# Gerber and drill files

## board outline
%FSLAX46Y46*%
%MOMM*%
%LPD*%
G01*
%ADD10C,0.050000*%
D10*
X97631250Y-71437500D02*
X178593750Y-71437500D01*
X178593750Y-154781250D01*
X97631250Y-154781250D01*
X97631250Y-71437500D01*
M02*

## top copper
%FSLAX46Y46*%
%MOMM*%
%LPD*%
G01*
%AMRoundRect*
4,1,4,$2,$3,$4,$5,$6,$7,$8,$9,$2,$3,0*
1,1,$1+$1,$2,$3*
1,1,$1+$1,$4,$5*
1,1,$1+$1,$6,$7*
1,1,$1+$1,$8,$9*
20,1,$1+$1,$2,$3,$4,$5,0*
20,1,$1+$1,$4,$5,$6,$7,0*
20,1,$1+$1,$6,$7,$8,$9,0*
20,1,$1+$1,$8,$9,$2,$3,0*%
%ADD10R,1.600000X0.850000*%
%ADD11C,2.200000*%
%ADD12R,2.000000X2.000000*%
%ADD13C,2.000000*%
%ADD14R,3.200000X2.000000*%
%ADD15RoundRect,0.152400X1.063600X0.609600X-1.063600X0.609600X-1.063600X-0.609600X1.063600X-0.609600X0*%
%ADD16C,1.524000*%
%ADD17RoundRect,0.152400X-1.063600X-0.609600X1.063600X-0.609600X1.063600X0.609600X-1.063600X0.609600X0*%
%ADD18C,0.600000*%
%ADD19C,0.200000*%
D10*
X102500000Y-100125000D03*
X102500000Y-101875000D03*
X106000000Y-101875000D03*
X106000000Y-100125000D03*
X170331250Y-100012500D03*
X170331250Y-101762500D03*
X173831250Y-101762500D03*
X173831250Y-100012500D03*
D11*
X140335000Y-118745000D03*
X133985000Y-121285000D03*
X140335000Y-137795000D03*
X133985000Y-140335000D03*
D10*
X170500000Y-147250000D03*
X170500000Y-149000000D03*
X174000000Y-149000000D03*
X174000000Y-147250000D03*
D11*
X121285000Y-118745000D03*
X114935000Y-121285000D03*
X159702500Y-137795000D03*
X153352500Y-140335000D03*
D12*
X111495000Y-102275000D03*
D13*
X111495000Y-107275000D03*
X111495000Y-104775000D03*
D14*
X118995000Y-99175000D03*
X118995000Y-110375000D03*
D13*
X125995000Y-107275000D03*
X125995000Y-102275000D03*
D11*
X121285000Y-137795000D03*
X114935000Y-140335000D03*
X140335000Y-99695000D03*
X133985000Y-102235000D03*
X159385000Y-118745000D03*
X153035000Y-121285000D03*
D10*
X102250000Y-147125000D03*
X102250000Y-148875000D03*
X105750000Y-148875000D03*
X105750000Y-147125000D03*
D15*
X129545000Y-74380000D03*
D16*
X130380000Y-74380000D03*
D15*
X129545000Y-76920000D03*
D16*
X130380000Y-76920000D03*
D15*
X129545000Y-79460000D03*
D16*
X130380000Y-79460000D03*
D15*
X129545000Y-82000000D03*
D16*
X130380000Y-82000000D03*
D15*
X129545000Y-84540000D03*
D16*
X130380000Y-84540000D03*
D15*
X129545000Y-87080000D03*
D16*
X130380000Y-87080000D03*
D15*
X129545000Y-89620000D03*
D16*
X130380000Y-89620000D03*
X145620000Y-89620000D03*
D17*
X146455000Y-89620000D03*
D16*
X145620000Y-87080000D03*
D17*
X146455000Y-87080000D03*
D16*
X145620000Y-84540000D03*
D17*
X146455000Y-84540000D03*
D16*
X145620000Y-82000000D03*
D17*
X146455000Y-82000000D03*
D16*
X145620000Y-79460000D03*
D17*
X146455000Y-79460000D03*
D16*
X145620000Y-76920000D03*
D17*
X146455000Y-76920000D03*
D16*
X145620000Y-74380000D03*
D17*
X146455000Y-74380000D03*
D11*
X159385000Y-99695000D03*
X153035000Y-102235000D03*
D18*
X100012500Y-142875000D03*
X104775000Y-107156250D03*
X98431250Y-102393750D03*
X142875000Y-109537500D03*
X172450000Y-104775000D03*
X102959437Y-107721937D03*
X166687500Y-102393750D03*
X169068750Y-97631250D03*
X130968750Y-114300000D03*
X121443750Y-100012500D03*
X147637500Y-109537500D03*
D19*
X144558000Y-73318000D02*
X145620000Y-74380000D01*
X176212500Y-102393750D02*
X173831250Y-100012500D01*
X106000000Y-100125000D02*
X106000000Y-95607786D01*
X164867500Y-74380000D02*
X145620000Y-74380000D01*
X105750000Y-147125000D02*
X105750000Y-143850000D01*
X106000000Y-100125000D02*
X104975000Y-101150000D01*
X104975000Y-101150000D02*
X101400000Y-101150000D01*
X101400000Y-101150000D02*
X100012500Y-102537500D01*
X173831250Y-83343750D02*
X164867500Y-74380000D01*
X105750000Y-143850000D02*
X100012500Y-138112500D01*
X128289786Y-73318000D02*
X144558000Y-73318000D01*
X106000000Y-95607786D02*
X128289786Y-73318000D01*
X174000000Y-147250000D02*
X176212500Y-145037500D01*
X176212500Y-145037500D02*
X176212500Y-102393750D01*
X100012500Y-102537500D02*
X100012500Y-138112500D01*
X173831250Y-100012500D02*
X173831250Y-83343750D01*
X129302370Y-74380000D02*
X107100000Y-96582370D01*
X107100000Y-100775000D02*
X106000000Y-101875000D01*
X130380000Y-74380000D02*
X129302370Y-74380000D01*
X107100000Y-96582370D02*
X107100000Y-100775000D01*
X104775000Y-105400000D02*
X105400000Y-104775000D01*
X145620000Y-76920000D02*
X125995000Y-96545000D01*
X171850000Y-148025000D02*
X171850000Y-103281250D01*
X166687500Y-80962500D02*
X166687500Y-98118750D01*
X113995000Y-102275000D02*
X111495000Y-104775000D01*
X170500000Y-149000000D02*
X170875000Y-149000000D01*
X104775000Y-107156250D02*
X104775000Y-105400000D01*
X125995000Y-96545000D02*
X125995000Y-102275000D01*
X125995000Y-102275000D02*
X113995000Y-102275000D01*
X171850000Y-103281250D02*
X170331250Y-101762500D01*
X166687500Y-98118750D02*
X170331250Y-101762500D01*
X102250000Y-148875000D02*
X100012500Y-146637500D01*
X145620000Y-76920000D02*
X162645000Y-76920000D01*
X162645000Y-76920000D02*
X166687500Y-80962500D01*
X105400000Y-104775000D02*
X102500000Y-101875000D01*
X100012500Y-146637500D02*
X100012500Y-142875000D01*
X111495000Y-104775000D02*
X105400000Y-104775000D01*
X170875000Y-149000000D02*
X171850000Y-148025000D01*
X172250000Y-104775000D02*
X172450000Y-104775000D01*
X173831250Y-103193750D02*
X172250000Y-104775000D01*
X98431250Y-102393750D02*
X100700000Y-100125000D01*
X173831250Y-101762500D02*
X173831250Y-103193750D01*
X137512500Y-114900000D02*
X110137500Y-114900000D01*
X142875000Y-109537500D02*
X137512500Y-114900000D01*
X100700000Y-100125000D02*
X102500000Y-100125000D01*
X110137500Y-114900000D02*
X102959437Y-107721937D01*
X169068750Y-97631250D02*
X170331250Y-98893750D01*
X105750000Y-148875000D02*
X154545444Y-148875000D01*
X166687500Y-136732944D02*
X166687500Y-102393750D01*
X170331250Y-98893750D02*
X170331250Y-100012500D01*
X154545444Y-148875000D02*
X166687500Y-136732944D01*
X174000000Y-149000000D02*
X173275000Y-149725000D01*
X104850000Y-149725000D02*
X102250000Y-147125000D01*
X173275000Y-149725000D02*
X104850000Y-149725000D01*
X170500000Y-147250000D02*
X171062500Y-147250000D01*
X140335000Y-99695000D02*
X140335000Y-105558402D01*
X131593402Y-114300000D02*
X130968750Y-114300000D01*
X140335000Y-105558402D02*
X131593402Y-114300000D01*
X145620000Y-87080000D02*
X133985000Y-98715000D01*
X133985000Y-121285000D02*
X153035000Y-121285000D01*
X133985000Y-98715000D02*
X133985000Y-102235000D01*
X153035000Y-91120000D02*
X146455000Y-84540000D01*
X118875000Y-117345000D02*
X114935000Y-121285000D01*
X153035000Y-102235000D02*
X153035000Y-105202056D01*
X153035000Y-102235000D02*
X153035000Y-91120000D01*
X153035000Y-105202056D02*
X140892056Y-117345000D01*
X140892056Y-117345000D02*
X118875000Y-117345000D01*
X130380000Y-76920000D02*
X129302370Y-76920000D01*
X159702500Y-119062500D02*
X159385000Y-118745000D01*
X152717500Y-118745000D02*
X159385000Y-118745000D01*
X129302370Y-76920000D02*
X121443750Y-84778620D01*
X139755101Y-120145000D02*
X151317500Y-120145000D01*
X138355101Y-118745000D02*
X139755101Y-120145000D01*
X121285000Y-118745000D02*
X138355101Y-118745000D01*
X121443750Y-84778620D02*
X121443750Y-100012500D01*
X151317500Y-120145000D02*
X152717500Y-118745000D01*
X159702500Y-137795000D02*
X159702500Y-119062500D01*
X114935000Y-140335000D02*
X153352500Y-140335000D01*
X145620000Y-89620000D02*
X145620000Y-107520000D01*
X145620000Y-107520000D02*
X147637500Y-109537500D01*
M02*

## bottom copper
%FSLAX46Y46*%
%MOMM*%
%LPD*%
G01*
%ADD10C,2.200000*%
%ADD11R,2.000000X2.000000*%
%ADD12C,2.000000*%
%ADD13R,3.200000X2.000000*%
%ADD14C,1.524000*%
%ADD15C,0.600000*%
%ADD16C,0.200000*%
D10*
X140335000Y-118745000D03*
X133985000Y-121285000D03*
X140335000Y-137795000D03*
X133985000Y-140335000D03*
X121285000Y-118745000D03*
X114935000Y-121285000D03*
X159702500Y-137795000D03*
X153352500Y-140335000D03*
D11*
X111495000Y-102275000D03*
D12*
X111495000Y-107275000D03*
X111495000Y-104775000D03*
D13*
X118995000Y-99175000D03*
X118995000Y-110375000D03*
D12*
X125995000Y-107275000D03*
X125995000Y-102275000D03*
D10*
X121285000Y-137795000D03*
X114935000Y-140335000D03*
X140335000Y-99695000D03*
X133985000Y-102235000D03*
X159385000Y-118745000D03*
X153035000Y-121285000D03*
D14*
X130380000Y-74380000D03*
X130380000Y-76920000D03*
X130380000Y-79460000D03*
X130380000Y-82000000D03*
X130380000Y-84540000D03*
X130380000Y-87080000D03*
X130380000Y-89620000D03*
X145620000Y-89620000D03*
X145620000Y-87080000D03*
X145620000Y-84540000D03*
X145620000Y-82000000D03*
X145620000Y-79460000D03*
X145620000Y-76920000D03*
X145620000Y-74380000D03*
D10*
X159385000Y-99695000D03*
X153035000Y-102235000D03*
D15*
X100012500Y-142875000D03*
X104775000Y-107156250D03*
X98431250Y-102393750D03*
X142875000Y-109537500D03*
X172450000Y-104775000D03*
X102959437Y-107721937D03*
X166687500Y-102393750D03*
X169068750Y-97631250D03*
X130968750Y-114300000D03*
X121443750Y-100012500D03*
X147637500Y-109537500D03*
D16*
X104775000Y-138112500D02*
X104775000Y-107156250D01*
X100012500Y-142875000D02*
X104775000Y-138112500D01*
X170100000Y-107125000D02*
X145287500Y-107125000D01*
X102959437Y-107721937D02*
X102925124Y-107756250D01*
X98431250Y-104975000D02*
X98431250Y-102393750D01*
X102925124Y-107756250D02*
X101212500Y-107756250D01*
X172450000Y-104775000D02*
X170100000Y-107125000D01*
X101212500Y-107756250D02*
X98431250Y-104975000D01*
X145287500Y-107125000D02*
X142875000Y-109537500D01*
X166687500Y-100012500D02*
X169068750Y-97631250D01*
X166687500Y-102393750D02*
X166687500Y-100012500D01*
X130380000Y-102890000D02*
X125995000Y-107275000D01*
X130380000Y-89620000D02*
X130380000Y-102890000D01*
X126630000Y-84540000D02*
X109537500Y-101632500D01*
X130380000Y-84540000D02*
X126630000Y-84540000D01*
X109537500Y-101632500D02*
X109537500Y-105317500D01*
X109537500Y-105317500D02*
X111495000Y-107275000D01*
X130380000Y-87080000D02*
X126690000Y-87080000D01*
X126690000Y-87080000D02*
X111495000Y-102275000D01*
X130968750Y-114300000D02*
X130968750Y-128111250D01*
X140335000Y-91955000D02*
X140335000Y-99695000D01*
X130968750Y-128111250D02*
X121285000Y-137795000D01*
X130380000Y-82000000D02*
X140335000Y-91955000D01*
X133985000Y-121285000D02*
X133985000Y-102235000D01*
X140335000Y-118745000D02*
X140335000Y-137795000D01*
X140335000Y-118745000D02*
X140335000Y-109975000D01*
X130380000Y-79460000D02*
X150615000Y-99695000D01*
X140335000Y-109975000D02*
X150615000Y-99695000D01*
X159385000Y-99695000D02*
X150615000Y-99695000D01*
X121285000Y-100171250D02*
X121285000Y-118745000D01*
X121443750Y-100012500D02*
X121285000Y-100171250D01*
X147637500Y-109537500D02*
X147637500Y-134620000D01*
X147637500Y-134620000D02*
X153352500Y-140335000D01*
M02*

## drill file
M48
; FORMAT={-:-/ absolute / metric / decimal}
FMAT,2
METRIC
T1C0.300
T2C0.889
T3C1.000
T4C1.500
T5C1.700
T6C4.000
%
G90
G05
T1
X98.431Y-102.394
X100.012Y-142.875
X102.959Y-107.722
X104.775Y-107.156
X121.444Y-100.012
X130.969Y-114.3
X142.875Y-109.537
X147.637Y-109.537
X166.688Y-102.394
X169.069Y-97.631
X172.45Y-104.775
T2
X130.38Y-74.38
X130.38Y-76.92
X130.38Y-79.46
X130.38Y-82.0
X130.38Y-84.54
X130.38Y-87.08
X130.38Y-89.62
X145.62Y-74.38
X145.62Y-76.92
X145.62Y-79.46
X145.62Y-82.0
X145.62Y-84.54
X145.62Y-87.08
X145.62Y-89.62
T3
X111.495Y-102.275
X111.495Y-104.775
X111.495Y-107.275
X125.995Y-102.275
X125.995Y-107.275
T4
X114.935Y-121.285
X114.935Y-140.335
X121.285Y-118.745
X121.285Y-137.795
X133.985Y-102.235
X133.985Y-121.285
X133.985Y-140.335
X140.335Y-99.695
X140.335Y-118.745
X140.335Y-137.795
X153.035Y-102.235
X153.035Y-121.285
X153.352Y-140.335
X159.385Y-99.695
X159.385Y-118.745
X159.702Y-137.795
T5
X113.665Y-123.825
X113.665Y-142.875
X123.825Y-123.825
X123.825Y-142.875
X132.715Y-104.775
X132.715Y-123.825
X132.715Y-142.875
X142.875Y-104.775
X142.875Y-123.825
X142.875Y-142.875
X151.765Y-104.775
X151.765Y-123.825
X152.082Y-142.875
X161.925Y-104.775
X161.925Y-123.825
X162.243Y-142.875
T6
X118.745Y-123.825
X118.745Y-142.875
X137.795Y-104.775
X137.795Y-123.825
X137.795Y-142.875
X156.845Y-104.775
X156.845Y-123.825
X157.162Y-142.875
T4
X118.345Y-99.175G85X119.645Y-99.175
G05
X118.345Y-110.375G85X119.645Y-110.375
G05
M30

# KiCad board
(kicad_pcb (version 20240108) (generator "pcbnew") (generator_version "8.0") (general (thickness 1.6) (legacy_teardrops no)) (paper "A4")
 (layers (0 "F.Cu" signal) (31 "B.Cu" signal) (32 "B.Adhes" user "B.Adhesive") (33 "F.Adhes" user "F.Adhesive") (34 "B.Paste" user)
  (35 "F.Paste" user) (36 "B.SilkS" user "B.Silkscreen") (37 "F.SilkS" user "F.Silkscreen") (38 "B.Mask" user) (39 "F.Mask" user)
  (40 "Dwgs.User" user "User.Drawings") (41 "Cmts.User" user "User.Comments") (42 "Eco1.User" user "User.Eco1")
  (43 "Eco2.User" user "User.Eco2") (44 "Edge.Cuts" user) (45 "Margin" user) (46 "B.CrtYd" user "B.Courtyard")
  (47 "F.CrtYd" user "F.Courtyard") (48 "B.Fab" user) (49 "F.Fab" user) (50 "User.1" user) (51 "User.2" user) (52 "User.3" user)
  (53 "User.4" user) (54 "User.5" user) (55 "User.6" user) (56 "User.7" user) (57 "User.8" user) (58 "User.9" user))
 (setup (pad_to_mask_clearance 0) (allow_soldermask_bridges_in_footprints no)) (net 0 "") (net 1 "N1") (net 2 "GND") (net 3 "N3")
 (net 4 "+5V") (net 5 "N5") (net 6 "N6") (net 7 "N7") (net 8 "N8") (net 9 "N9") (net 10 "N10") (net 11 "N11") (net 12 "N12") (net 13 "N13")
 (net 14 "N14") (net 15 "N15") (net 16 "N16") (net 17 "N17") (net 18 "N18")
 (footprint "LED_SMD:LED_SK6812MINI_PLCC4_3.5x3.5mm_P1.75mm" (layer "F.Cu") (at 104.25 101)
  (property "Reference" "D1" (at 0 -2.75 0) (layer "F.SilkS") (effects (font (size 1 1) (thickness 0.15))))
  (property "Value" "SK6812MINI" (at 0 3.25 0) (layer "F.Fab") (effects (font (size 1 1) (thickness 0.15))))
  (pad "1" smd rect (at -1.75 -0.875) (size 1.6 0.85) (layers "F.Cu" "F.Paste" "F.Mask") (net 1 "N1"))
  (pad "2" smd rect (at -1.75 0.875) (size 1.6 0.85) (layers "F.Cu" "F.Paste" "F.Mask") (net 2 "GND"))
  (pad "3" smd rect (at 1.75 0.875) (size 1.6 0.85) (layers "F.Cu" "F.Paste" "F.Mask") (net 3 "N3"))
  (pad "4" smd rect (at 1.75 -0.875) (size 1.6 0.85) (layers "F.Cu" "F.Paste" "F.Mask") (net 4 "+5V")))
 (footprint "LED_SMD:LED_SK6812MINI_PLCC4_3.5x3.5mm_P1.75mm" (layer "F.Cu") (at 172.08125 100.8875)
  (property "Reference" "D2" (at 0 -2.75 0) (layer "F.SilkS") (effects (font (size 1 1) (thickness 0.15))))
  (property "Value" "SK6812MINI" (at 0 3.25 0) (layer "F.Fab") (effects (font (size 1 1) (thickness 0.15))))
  (pad "1" smd rect (at -1.75 -0.875) (size 1.6 0.85) (layers "F.Cu" "F.Paste" "F.Mask") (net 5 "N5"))
  (pad "2" smd rect (at -1.75 0.875) (size 1.6 0.85) (layers "F.Cu" "F.Paste" "F.Mask") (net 2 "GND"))
  (pad "3" smd rect (at 1.75 0.875) (size 1.6 0.85) (layers "F.Cu" "F.Paste" "F.Mask") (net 1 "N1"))
  (pad "4" smd rect (at 1.75 -0.875) (size 1.6 0.85) (layers "F.Cu" "F.Paste" "F.Mask") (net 4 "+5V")))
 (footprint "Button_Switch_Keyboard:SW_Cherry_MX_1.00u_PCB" (layer "F.Cu") (at 140.335 118.745)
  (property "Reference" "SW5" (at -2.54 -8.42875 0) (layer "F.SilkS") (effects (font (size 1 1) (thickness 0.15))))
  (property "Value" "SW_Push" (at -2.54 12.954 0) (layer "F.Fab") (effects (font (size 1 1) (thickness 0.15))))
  (pad "" np_thru_hole circle (at -7.62 5.08) (size 1.7 1.7) (drill 1.7) (layers "*.Cu" "*.Mask"))
  (pad "" np_thru_hole circle (at -2.54 5.08) (size 4 4) (drill 4) (layers "*.Cu" "*.Mask"))
  (pad "" np_thru_hole circle (at 2.54 5.08) (size 1.7 1.7) (drill 1.7) (layers "*.Cu" "*.Mask"))
  (pad "1" thru_hole circle (at 0 0) (size 2.2 2.2) (drill 1.5) (layers "*.Cu" "*.Mask") (remove_unused_layers no) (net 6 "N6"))
  (pad "2" thru_hole circle (at -6.35 2.54) (size 2.2 2.2) (drill 1.5) (layers "*.Cu" "*.Mask") (remove_unused_layers no) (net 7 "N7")))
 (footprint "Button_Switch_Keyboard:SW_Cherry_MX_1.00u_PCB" (layer "F.Cu") (at 140.335 137.795)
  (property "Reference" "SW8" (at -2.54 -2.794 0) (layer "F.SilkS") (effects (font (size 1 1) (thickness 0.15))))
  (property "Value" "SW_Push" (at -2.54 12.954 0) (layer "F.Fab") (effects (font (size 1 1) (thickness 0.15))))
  (pad "" np_thru_hole circle (at -7.62 5.08) (size 1.7 1.7) (drill 1.7) (layers "*.Cu" "*.Mask"))
  (pad "" np_thru_hole circle (at -2.54 5.08) (size 4 4) (drill 4) (layers "*.Cu" "*.Mask"))
  (pad "" np_thru_hole circle (at 2.54 5.08) (size 1.7 1.7) (drill 1.7) (layers "*.Cu" "*.Mask"))
  (pad "1" thru_hole circle (at 0 0) (size 2.2 2.2) (drill 1.5) (layers "*.Cu" "*.Mask") (remove_unused_layers no) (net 6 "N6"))
  (pad "2" thru_hole circle (at -6.35 2.54) (size 2.2 2.2) (drill 1.5) (layers "*.Cu" "*.Mask") (remove_unused_layers no) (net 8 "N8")))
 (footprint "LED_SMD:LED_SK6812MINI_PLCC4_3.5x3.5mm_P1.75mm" (layer "F.Cu") (at 172.25 148.125)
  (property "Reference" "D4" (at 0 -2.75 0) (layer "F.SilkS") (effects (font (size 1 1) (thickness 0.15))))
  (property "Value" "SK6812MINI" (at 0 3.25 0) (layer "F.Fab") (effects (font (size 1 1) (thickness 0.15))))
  (pad "1" smd rect (at -1.75 -0.875) (size 1.6 0.85) (layers "F.Cu" "F.Paste" "F.Mask") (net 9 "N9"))
  (pad "2" smd rect (at -1.75 0.875) (size 1.6 0.85) (layers "F.Cu" "F.Paste" "F.Mask") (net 2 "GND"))
  (pad "3" smd rect (at 1.75 0.875) (size 1.6 0.85) (layers "F.Cu" "F.Paste" "F.Mask") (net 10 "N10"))
  (pad "4" smd rect (at 1.75 -0.875) (size 1.6 0.85) (layers "F.Cu" "F.Paste" "F.Mask") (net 4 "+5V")))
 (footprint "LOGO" (layer "F.Cu") (at 161.925 83.34375)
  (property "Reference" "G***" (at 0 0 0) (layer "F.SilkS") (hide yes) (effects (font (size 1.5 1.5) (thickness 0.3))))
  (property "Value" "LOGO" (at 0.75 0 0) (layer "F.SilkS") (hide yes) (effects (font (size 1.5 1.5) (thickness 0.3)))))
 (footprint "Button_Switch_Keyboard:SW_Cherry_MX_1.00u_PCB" (layer "F.Cu") (at 121.285 118.745)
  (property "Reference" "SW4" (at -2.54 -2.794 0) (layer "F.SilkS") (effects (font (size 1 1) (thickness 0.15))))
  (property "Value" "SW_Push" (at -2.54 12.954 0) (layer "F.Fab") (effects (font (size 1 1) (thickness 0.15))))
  (pad "" np_thru_hole circle (at -7.62 5.08) (size 1.7 1.7) (drill 1.7) (layers "*.Cu" "*.Mask"))
  (pad "" np_thru_hole circle (at -2.54 5.08) (size 4 4) (drill 4) (layers "*.Cu" "*.Mask"))
  (pad "" np_thru_hole circle (at 2.54 5.08) (size 1.7 1.7) (drill 1.7) (layers "*.Cu" "*.Mask"))
  (pad "1" thru_hole circle (at 0 0) (size 2.2 2.2) (drill 1.5) (layers "*.Cu" "*.Mask") (remove_unused_layers no) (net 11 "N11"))
  (pad "2" thru_hole circle (at -6.35 2.54) (size 2.2 2.2) (drill 1.5) (layers "*.Cu" "*.Mask") (remove_unused_layers no) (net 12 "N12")))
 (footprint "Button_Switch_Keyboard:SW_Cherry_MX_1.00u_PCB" (layer "F.Cu") (at 159.7025 137.795)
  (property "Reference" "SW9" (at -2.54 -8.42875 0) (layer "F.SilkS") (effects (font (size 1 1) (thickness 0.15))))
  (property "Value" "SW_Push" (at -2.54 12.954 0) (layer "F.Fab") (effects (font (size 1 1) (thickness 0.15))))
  (pad "" np_thru_hole circle (at -7.62 5.08) (size 1.7 1.7) (drill 1.7) (layers "*.Cu" "*.Mask"))
  (pad "" np_thru_hole circle (at -2.54 5.08) (size 4 4) (drill 4) (layers "*.Cu" "*.Mask"))
  (pad "" np_thru_hole circle (at 2.54 5.08) (size 1.7 1.7) (drill 1.7) (layers "*.Cu" "*.Mask"))
  (pad "1" thru_hole circle (at 0 0) (size 2.2 2.2) (drill 1.5) (layers "*.Cu" "*.Mask") (remove_unused_layers no) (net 11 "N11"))
  (pad "2" thru_hole circle (at -6.35 2.54) (size 2.2 2.2) (drill 1.5) (layers "*.Cu" "*.Mask") (remove_unused_layers no) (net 8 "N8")))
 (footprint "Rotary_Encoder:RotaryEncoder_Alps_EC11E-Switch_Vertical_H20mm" (layer "F.Cu") (at 111.495 102.275)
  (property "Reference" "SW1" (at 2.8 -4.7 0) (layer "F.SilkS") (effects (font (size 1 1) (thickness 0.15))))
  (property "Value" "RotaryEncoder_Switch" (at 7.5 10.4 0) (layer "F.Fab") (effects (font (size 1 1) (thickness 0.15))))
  (pad "A" thru_hole rect (at 0 0) (size 2 2) (drill 1) (layers "*.Cu" "*.Mask") (remove_unused_layers no) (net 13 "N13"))
  (pad "B" thru_hole circle (at 0 5) (size 2 2) (drill 1) (layers "*.Cu" "*.Mask") (remove_unused_layers no) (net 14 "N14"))
  (pad "C" thru_hole circle (at 0 2.5) (size 2 2) (drill 1) (layers "*.Cu" "*.Mask") (remove_unused_layers no) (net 2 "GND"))
  (pad "MP" thru_hole rect (at 7.5 -3.1) (size 3.2 2) (drill oval 2.8 1.5) (layers "*.Cu" "*.Mask") (remove_unused_layers no))
  (pad "MP" thru_hole rect (at 7.5 8.1) (size 3.2 2) (drill oval 2.8 1.5) (layers "*.Cu" "*.Mask") (remove_unused_layers no))
  (pad "S1" thru_hole circle (at 14.5 5) (size 2 2) (drill 1) (layers "*.Cu" "*.Mask") (remove_unused_layers no) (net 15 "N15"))
  (pad "S2" thru_hole circle (at 14.5 0) (size 2 2) (drill 1) (layers "*.Cu" "*.Mask") (remove_unused_layers no) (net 2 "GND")))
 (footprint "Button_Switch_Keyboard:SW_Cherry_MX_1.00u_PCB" (layer "F.Cu") (at 121.285 137.795)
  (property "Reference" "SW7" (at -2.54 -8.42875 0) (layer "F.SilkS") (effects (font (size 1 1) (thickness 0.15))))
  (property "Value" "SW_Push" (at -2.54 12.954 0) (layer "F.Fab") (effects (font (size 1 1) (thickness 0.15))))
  (pad "" np_thru_hole circle (at -7.62 5.08) (size 1.7 1.7) (drill 1.7) (layers "*.Cu" "*.Mask"))
  (pad "" np_thru_hole circle (at -2.54 5.08) (size 4 4) (drill 4) (layers "*.Cu" "*.Mask"))
  (pad "" np_thru_hole circle (at 2.54 5.08) (size 1.7 1.7) (drill 1.7) (layers "*.Cu" "*.Mask"))
  (pad "1" thru_hole circle (at 0 0) (size 2.2 2.2) (drill 1.5) (layers "*.Cu" "*.Mask") (remove_unused_layers no) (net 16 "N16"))
  (pad "2" thru_hole circle (at -6.35 2.54) (size 2.2 2.2) (drill 1.5) (layers "*.Cu" "*.Mask") (remove_unused_layers no) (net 8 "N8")))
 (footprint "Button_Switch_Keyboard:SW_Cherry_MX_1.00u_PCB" (layer "F.Cu") (at 140.335 99.695)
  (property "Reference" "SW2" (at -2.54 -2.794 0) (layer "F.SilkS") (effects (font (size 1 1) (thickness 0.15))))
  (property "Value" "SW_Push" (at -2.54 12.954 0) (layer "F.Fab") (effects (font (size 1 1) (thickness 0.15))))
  (pad "" np_thru_hole circle (at -7.62 5.08) (size 1.7 1.7) (drill 1.7) (layers "*.Cu" "*.Mask"))
  (pad "" np_thru_hole circle (at -2.54 5.08) (size 4 4) (drill 4) (layers "*.Cu" "*.Mask"))
  (pad "" np_thru_hole circle (at 2.54 5.08) (size 1.7 1.7) (drill 1.7) (layers "*.Cu" "*.Mask"))
  (pad "1" thru_hole circle (at 0 0) (size 2.2 2.2) (drill 1.5) (layers "*.Cu" "*.Mask") (remove_unused_layers no) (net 16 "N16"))
  (pad "2" thru_hole circle (at -6.35 2.54) (size 2.2 2.2) (drill 1.5) (layers "*.Cu" "*.Mask") (remove_unused_layers no) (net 7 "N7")))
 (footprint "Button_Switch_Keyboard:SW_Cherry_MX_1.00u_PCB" (layer "F.Cu") (at 159.385 118.745)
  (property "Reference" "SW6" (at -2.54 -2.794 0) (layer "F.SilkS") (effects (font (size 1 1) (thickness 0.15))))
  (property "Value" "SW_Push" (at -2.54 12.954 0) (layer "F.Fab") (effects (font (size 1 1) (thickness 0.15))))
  (pad "" np_thru_hole circle (at -7.62 5.08) (size 1.7 1.7) (drill 1.7) (layers "*.Cu" "*.Mask"))
  (pad "" np_thru_hole circle (at -2.54 5.08) (size 4 4) (drill 4) (layers "*.Cu" "*.Mask"))
  (pad "" np_thru_hole circle (at 2.54 5.08) (size 1.7 1.7) (drill 1.7) (layers "*.Cu" "*.Mask"))
  (pad "1" thru_hole circle (at 0 0) (size 2.2 2.2) (drill 1.5) (layers "*.Cu" "*.Mask") (remove_unused_layers no) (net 11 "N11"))
  (pad "2" thru_hole circle (at -6.35 2.54) (size 2.2 2.2) (drill 1.5) (layers "*.Cu" "*.Mask") (remove_unused_layers no) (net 7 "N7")))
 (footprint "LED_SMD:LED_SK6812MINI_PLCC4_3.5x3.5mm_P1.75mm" (layer "F.Cu") (at 104 148)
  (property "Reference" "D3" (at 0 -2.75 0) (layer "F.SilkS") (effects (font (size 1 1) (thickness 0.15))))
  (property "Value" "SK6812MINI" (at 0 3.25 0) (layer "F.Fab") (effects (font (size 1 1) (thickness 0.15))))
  (pad "1" smd rect (at -1.75 -0.875) (size 1.6 0.85) (layers "F.Cu" "F.Paste" "F.Mask") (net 10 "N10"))
  (pad "2" smd rect (at -1.75 0.875) (size 1.6 0.85) (layers "F.Cu" "F.Paste" "F.Mask") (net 2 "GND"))
  (pad "3" smd rect (at 1.75 0.875) (size 1.6 0.85) (layers "F.Cu" "F.Paste" "F.Mask") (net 5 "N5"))
  (pad "4" smd rect (at 1.75 -0.875) (size 1.6 0.85) (layers "F.Cu" "F.Paste" "F.Mask") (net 4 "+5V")))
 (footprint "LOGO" (layer "F.Cu") (at 111.91875 83.34375 -90)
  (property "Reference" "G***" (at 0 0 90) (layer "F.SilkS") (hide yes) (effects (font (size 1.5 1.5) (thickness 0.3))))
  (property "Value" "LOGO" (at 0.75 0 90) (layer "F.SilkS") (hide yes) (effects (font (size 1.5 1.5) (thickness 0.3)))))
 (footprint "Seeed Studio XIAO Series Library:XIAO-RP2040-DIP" (layer "F.Cu") (at 138 82)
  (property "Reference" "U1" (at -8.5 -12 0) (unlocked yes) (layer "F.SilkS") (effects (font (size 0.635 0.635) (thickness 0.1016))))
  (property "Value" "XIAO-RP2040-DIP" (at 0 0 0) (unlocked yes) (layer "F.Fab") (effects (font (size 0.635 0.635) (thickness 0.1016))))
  (pad "1" smd roundrect (at -8.455 -7.62 180) (size 2.432 1.524) (layers "F.Cu" "F.Mask") (roundrect_rratio 0.1) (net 3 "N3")
   (thermal_bridge_angle 45))
  (pad "1" thru_hole circle (at -7.62 -7.62 180) (size 1.524 1.524) (drill 0.889) (layers "*.Cu" "*.Mask") (remove_unused_layers no)
   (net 3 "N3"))
  (pad "2" smd roundrect (at -8.455 -5.08 180) (size 2.432 1.524) (layers "F.Cu" "F.Mask") (roundrect_rratio 0.1) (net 11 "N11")
   (thermal_bridge_angle 45))
  (pad "2" thru_hole circle (at -7.62 -5.08 180) (size 1.524 1.524) (drill 0.889) (layers "*.Cu" "*.Mask") (remove_unused_layers no)
   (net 11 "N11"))
  (pad "3" smd roundrect (at -8.455 -2.54 180) (size 2.432 1.524) (layers "F.Cu" "F.Mask") (roundrect_rratio 0.1) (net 6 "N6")
   (thermal_bridge_angle 45))
  (pad "3" thru_hole circle (at -7.62 -2.54 180) (size 1.524 1.524) (drill 0.889) (layers "*.Cu" "*.Mask") (remove_unused_layers no)
   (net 6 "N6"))
  (pad "4" smd roundrect (at -8.455 0 180) (size 2.432 1.524) (layers "F.Cu" "F.Mask") (roundrect_rratio 0.1) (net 16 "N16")
   (thermal_bridge_angle 45))
  (pad "4" thru_hole circle (at -7.62 0 180) (size 1.524 1.524) (drill 0.889) (layers "*.Cu" "*.Mask") (remove_unused_layers no)
   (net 16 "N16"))
  (pad "5" smd roundrect (at -8.455 2.54 180) (size 2.432 1.524) (layers "F.Cu" "F.Mask") (roundrect_rratio 0.1) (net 14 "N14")
   (thermal_bridge_angle 45))
  (pad "5" thru_hole circle (at -7.62 2.54 180) (size 1.524 1.524) (drill 0.889) (layers "*.Cu" "*.Mask") (remove_unused_layers no)
   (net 14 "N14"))
  (pad "6" smd roundrect (at -8.455 5.08 180) (size 2.432 1.524) (layers "F.Cu" "F.Mask") (roundrect_rratio 0.1) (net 13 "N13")
   (thermal_bridge_angle 45))
  (pad "6" thru_hole circle (at -7.62 5.08 180) (size 1.524 1.524) (drill 0.889) (layers "*.Cu" "*.Mask") (remove_unused_layers no)
   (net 13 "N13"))
  (pad "7" smd roundrect (at -8.455 7.62 180) (size 2.432 1.524) (layers "F.Cu" "F.Mask") (roundrect_rratio 0.1) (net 15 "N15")
   (thermal_bridge_angle 45))
  (pad "7" thru_hole circle (at -7.62 7.62 180) (size 1.524 1.524) (drill 0.889) (layers "*.Cu" "*.Mask") (remove_unused_layers no)
   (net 15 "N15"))
  (pad "8" thru_hole circle (at 7.62 7.62) (size 1.524 1.524) (drill 0.889) (layers "*.Cu" "*.Mask") (remove_unused_layers no) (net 8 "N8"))
  (pad "8" smd roundrect (at 8.455 7.62) (size 2.432 1.524) (layers "F.Cu" "F.Mask") (roundrect_rratio 0.1) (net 8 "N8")
   (thermal_bridge_angle 45))
  (pad "9" thru_hole circle (at 7.62 5.08) (size 1.524 1.524) (drill 0.889) (layers "*.Cu" "*.Mask") (remove_unused_layers no) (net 7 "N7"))
  (pad "9" smd roundrect (at 8.455 5.08) (size 2.432 1.524) (layers "F.Cu" "F.Mask") (roundrect_rratio 0.1) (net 7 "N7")
   (thermal_bridge_angle 45))
  (pad "10" thru_hole circle (at 7.62 2.54) (size 1.524 1.524) (drill 0.889) (layers "*.Cu" "*.Mask") (remove_unused_layers no)
   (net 12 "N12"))
  (pad "10" smd roundrect (at 8.455 2.54) (size 2.432 1.524) (layers "F.Cu" "F.Mask") (roundrect_rratio 0.1) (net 12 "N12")
   (thermal_bridge_angle 45))
  (pad "11" thru_hole circle (at 7.62 0) (size 1.524 1.524) (drill 0.889) (layers "*.Cu" "*.Mask") (remove_unused_layers no) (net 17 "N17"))
  (pad "11" smd roundrect (at 8.455 0) (size 2.432 1.524) (layers "F.Cu" "F.Mask") (roundrect_rratio 0.1) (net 17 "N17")
   (thermal_bridge_angle 45))
  (pad "12" thru_hole circle (at 7.62 -2.54) (size 1.524 1.524) (drill 0.889) (layers "*.Cu" "*.Mask") (remove_unused_layers no)
   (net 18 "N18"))
  (pad "12" smd roundrect (at 8.455 -2.54) (size 2.432 1.524) (layers "F.Cu" "F.Mask") (roundrect_rratio 0.1) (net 18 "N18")
   (thermal_bridge_angle 45))
  (pad "13" thru_hole circle (at 7.62 -5.08) (size 1.524 1.524) (drill 0.889) (layers "*.Cu" "*.Mask") (remove_unused_layers no)
   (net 2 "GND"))
  (pad "13" smd roundrect (at 8.455 -5.08) (size 2.432 1.524) (layers "F.Cu" "F.Mask") (roundrect_rratio 0.1) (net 2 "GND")
   (thermal_bridge_angle 45))
  (pad "14" thru_hole circle (at 7.62 -7.62) (size 1.524 1.524) (drill 0.889) (layers "*.Cu" "*.Mask") (remove_unused_layers no)
   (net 4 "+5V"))
  (pad "14" smd roundrect (at 8.455 -7.62) (size 2.432 1.524) (layers "F.Cu" "F.Mask") (roundrect_rratio 0.1) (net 4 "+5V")
   (thermal_bridge_angle 45)))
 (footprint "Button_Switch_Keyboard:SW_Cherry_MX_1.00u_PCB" (layer "F.Cu") (at 159.385 99.695)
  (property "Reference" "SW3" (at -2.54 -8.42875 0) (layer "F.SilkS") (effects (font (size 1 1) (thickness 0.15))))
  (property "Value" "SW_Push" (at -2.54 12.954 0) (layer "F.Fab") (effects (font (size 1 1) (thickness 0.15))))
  (pad "" np_thru_hole circle (at -7.62 5.08) (size 1.7 1.7) (drill 1.7) (layers "*.Cu" "*.Mask"))
  (pad "" np_thru_hole circle (at -2.54 5.08) (size 4 4) (drill 4) (layers "*.Cu" "*.Mask"))
  (pad "" np_thru_hole circle (at 2.54 5.08) (size 1.7 1.7) (drill 1.7) (layers "*.Cu" "*.Mask"))
  (pad "1" thru_hole circle (at 0 0) (size 2.2 2.2) (drill 1.5) (layers "*.Cu" "*.Mask") (remove_unused_layers no) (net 6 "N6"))
  (pad "2" thru_hole circle (at -6.35 2.54) (size 2.2 2.2) (drill 1.5) (layers "*.Cu" "*.Mask") (remove_unused_layers no) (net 12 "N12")))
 (gr_rect (start 97.63125 71.4375) (end 178.59375 154.78125) (stroke (width 0.05) (type default)) (fill none) (layer "Edge.Cuts"))
 (segment (start 144.558 73.318) (end 145.62 74.38) (width 0.2) (layer "F.Cu") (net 4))
 (segment (start 176.2125 102.39375) (end 173.83125 100.0125) (width 0.2) (layer "F.Cu") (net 4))
 (segment (start 106 100.125) (end 106 95.607786) (width 0.2) (layer "F.Cu") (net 4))
 (segment (start 164.8675 74.38) (end 145.62 74.38) (width 0.2) (layer "F.Cu") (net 4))
 (segment (start 105.75 147.125) (end 105.75 143.85) (width 0.2) (layer "F.Cu") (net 4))
 (segment (start 106 100.125) (end 104.975 101.15) (width 0.2) (layer "F.Cu") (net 4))
 (segment (start 104.975 101.15) (end 101.4 101.15) (width 0.2) (layer "F.Cu") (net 4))
 (segment (start 101.4 101.15) (end 100.0125 102.5375) (width 0.2) (layer "F.Cu") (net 4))
 (segment (start 173.83125 83.34375) (end 164.8675 74.38) (width 0.2) (layer "F.Cu") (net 4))
 (segment (start 105.75 143.85) (end 100.0125 138.1125) (width 0.2) (layer "F.Cu") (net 4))
 (segment (start 128.289786 73.318) (end 144.558 73.318) (width 0.2) (layer "F.Cu") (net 4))
 (segment (start 106 95.607786) (end 128.289786 73.318) (width 0.2) (layer "F.Cu") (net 4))
 (segment (start 174 147.25) (end 176.2125 145.0375) (width 0.2) (layer "F.Cu") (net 4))
 (segment (start 176.2125 145.0375) (end 176.2125 102.39375) (width 0.2) (layer "F.Cu") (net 4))
 (segment (start 100.0125 102.5375) (end 100.0125 138.1125) (width 0.2) (layer "F.Cu") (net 4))
 (segment (start 173.83125 100.0125) (end 173.83125 83.34375) (width 0.2) (layer "F.Cu") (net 4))
 (segment (start 129.30237 74.38) (end 107.1 96.58237) (width 0.2) (layer "F.Cu") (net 3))
 (segment (start 107.1 100.775) (end 106 101.875) (width 0.2) (layer "F.Cu") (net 3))
 (segment (start 130.38 74.38) (end 129.30237 74.38) (width 0.2) (layer "F.Cu") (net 3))
 (segment (start 107.1 96.58237) (end 107.1 100.775) (width 0.2) (layer "F.Cu") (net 3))
 (segment (start 104.775 105.4) (end 105.4 104.775) (width 0.2) (layer "F.Cu") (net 2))
 (segment (start 145.62 76.92) (end 125.995 96.545) (width 0.2) (layer "F.Cu") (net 2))
 (segment (start 171.85 148.025) (end 171.85 103.28125) (width 0.2) (layer "F.Cu") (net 2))
 (segment (start 166.6875 80.9625) (end 166.6875 98.11875) (width 0.2) (layer "F.Cu") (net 2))
 (segment (start 113.995 102.275) (end 111.495 104.775) (width 0.2) (layer "F.Cu") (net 2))
 (segment (start 170.5 149) (end 170.875 149) (width 0.2) (layer "F.Cu") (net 2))
 (segment (start 104.775 107.15625) (end 104.775 105.4) (width 0.2) (layer "F.Cu") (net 2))
 (segment (start 125.995 96.545) (end 125.995 102.275) (width 0.2) (layer "F.Cu") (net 2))
 (segment (start 125.995 102.275) (end 113.995 102.275) (width 0.2) (layer "F.Cu") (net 2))
 (segment (start 171.85 103.28125) (end 170.33125 101.7625) (width 0.2) (layer "F.Cu") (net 2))
 (segment (start 166.6875 98.11875) (end 170.33125 101.7625) (width 0.2) (layer "F.Cu") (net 2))
 (segment (start 102.25 148.875) (end 100.0125 146.6375) (width 0.2) (layer "F.Cu") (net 2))
 (segment (start 145.62 76.92) (end 162.645 76.92) (width 0.2) (layer "F.Cu") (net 2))
 (segment (start 162.645 76.92) (end 166.6875 80.9625) (width 0.2) (layer "F.Cu") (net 2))
 (segment (start 105.4 104.775) (end 102.5 101.875) (width 0.2) (layer "F.Cu") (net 2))
 (segment (start 100.0125 146.6375) (end 100.0125 142.875) (width 0.2) (layer "F.Cu") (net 2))
 (segment (start 111.495 104.775) (end 105.4 104.775) (width 0.2) (layer "F.Cu") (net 2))
 (segment (start 170.875 149) (end 171.85 148.025) (width 0.2) (layer "F.Cu") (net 2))
 (via (at 100.0125 142.875) (size 0.6) (drill 0.3) (layers "F.Cu" "B.Cu") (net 2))
 (via (at 104.775 107.15625) (size 0.6) (drill 0.3) (layers "F.Cu" "B.Cu") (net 2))
 (segment (start 104.775 138.1125) (end 104.775 107.15625) (width 0.2) (layer "B.Cu") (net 2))
 (segment (start 100.0125 142.875) (end 104.775 138.1125) (width 0.2) (layer "B.Cu") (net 2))
 (segment (start 172.25 104.775) (end 172.45 104.775) (width 0.2) (layer "F.Cu") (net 1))
 (segment (start 173.83125 103.19375) (end 172.25 104.775) (width 0.2) (layer "F.Cu") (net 1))
 (segment (start 98.43125 102.39375) (end 100.7 100.125) (width 0.2) (layer "F.Cu") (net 1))
 (segment (start 173.83125 101.7625) (end 173.83125 103.19375) (width 0.2) (layer "F.Cu") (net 1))
 (segment (start 137.5125 114.9) (end 110.1375 114.9) (width 0.2) (layer "F.Cu") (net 1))
 (segment (start 142.875 109.5375) (end 137.5125 114.9) (width 0.2) (layer "F.Cu") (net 1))
 (segment (start 100.7 100.125) (end 102.5 100.125) (width 0.2) (layer "F.Cu") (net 1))
 (segment (start 110.1375 114.9) (end 102.959437 107.721937) (width 0.2) (layer "F.Cu") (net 1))
 (via (at 98.43125 102.39375) (size 0.6) (drill 0.3) (layers "F.Cu" "B.Cu") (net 1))
 (via (at 142.875 109.5375) (size 0.6) (drill 0.3) (layers "F.Cu" "B.Cu") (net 1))
 (via (at 172.45 104.775) (size 0.6) (drill 0.3) (layers "F.Cu" "B.Cu") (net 1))
 (via (at 102.959437 107.721937) (size 0.6) (drill 0.3) (layers "F.Cu" "B.Cu") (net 1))
 (segment (start 170.1 107.125) (end 145.2875 107.125) (width 0.2) (layer "B.Cu") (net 1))
 (segment (start 102.959437 107.721937) (end 102.925124 107.75625) (width 0.2) (layer "B.Cu") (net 1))
 (segment (start 98.43125 104.975) (end 98.43125 102.39375) (width 0.2) (layer "B.Cu") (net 1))
 (segment (start 102.925124 107.75625) (end 101.2125 107.75625) (width 0.2) (layer "B.Cu") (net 1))
 (segment (start 172.45 104.775) (end 170.1 107.125) (width 0.2) (layer "B.Cu") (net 1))
 (segment (start 101.2125 107.75625) (end 98.43125 104.975) (width 0.2) (layer "B.Cu") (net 1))
 (segment (start 145.2875 107.125) (end 142.875 109.5375) (width 0.2) (layer "B.Cu") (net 1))
 (segment (start 169.06875 97.63125) (end 170.33125 98.89375) (width 0.2) (layer "F.Cu") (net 5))
 (segment (start 105.75 148.875) (end 154.545444 148.875) (width 0.2) (layer "F.Cu") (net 5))
 (segment (start 166.6875 136.732944) (end 166.6875 102.39375) (width 0.2) (layer "F.Cu") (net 5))
 (segment (start 170.33125 98.89375) (end 170.33125 100.0125) (width 0.2) (layer "F.Cu") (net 5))
 (segment (start 154.545444 148.875) (end 166.6875 136.732944) (width 0.2) (layer "F.Cu") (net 5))
 (via (at 166.6875 102.39375) (size 0.6) (drill 0.3) (layers "F.Cu" "B.Cu") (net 5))
 (via (at 169.06875 97.63125) (size 0.6) (drill 0.3) (layers "F.Cu" "B.Cu") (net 5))
 (segment (start 166.6875 100.0125) (end 169.06875 97.63125) (width 0.2) (layer "B.Cu") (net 5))
 (segment (start 166.6875 102.39375) (end 166.6875 100.0125) (width 0.2) (layer "B.Cu") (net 5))
 (segment (start 174 149) (end 173.275 149.725) (width 0.2) (layer "F.Cu") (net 10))
 (segment (start 104.85 149.725) (end 102.25 147.125) (width 0.2) (layer "F.Cu") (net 10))
 (segment (start 173.275 149.725) (end 104.85 149.725) (width 0.2) (layer "F.Cu") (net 10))
 (segment (start 170.5 147.25) (end 171.0625 147.25) (width 0.2) (layer "F.Cu") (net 9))
 (segment (start 130.38 102.89) (end 125.995 107.275) (width 0.2) (layer "B.Cu") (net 15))
 (segment (start 130.38 89.62) (end 130.38 102.89) (width 0.2) (layer "B.Cu") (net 15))
 (segment (start 126.63 84.54) (end 109.5375 101.6325) (width 0.2) (layer "B.Cu") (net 14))
 (segment (start 130.38 84.54) (end 126.63 84.54) (width 0.2) (layer "B.Cu") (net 14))
 (segment (start 109.5375 101.6325) (end 109.5375 105.3175) (width 0.2) (layer "B.Cu") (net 14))
 (segment (start 109.5375 105.3175) (end 111.495 107.275) (width 0.2) (layer "B.Cu") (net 14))
 (segment (start 130.38 87.08) (end 126.69 87.08) (width 0.2) (layer "B.Cu") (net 13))
 (segment (start 126.69 87.08) (end 111.495 102.275) (width 0.2) (layer "B.Cu") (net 13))
 (segment (start 140.335 99.695) (end 140.335 105.558402) (width 0.2) (layer "F.Cu") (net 16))
 (segment (start 131.593402 114.3) (end 130.96875 114.3) (width 0.2) (layer "F.Cu") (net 16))
 (segment (start 140.335 105.558402) (end 131.593402 114.3) (width 0.2) (layer "F.Cu") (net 16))
 (via (at 130.96875 114.3) (size 0.6) (drill 0.3) (layers "F.Cu" "B.Cu") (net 16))
 (segment (start 130.96875 114.3) (end 130.96875 128.11125) (width 0.2) (layer "B.Cu") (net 16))
 (segment (start 140.335 91.955) (end 140.335 99.695) (width 0.2) (layer "B.Cu") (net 16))
 (segment (start 130.96875 128.11125) (end 121.285 137.795) (width 0.2) (layer "B.Cu") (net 16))
 (segment (start 130.38 82) (end 140.335 91.955) (width 0.2) (layer "B.Cu") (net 16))
 (segment (start 145.62 87.08) (end 133.985 98.715) (width 0.2) (layer "F.Cu") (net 7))
 (segment (start 133.985 121.285) (end 153.035 121.285) (width 0.2) (layer "F.Cu") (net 7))
 (segment (start 133.985 98.715) (end 133.985 102.235) (width 0.2) (layer "F.Cu") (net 7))
 (segment (start 133.985 121.285) (end 133.985 102.235) (width 0.2) (layer "B.Cu") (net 7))
 (segment (start 153.035 91.12) (end 146.455 84.54) (width 0.2) (layer "F.Cu") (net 12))
 (segment (start 118.875 117.345) (end 114.935 121.285) (width 0.2) (layer "F.Cu") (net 12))
 (segment (start 153.035 102.235) (end 153.035 105.202056) (width 0.2) (layer "F.Cu") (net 12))
 (segment (start 153.035 102.235) (end 153.035 91.12) (width 0.2) (layer "F.Cu") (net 12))
 (segment (start 153.035 105.202056) (end 140.892056 117.345) (width 0.2) (layer "F.Cu") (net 12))
 (segment (start 140.892056 117.345) (end 118.875 117.345) (width 0.2) (layer "F.Cu") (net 12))
 (segment (start 140.335 118.745) (end 140.335 137.795) (width 0.2) (layer "B.Cu") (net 6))
 (segment (start 140.335 118.745) (end 140.335 109.975) (width 0.2) (layer "B.Cu") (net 6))
 (segment (start 130.38 79.46) (end 150.615 99.695) (width 0.2) (layer "B.Cu") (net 6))
 (segment (start 140.335 109.975) (end 150.615 99.695) (width 0.2) (layer "B.Cu") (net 6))
 (segment (start 159.385 99.695) (end 150.615 99.695) (width 0.2) (layer "B.Cu") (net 6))
 (segment (start 130.38 76.92) (end 129.30237 76.92) (width 0.2) (layer "F.Cu") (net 11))
 (segment (start 159.7025 119.0625) (end 159.385 118.745) (width 0.2) (layer "F.Cu") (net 11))
 (segment (start 152.7175 118.745) (end 159.385 118.745) (width 0.2) (layer "F.Cu") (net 11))
 (segment (start 129.30237 76.92) (end 121.44375 84.77862) (width 0.2) (layer "F.Cu") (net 11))
 (segment (start 139.755101 120.145) (end 151.3175 120.145) (width 0.2) (layer "F.Cu") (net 11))
 (segment (start 138.355101 118.745) (end 139.755101 120.145) (width 0.2) (layer "F.Cu") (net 11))
 (segment (start 121.285 118.745) (end 138.355101 118.745) (width 0.2) (layer "F.Cu") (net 11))
 (segment (start 121.44375 84.77862) (end 121.44375 100.0125) (width 0.2) (layer "F.Cu") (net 11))
 (segment (start 151.3175 120.145) (end 152.7175 118.745) (width 0.2) (layer "F.Cu") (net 11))
 (segment (start 159.7025 137.795) (end 159.7025 119.0625) (width 0.2) (layer "F.Cu") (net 11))
 (via (at 121.44375 100.0125) (size 0.6) (drill 0.3) (layers "F.Cu" "B.Cu") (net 11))
 (segment (start 121.285 100.17125) (end 121.285 118.745) (width 0.2) (layer "B.Cu") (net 11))
 (segment (start 121.44375 100.0125) (end 121.285 100.17125) (width 0.2) (layer "B.Cu") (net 11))
 (segment (start 114.935 140.335) (end 153.3525 140.335) (width 0.2) (layer "F.Cu") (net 8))
 (segment (start 145.62 89.62) (end 145.62 107.52) (width 0.2) (layer "F.Cu") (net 8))
 (segment (start 145.62 107.52) (end 147.6375 109.5375) (width 0.2) (layer "F.Cu") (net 8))
 (via (at 147.6375 109.5375) (size 0.6) (drill 0.3) (layers "F.Cu" "B.Cu") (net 8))
 (segment (start 147.6375 109.5375) (end 147.6375 134.62) (width 0.2) (layer "B.Cu") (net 8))
 (segment (start 147.6375 134.62) (end 153.3525 140.335) (width 0.2) (layer "B.Cu") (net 8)))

